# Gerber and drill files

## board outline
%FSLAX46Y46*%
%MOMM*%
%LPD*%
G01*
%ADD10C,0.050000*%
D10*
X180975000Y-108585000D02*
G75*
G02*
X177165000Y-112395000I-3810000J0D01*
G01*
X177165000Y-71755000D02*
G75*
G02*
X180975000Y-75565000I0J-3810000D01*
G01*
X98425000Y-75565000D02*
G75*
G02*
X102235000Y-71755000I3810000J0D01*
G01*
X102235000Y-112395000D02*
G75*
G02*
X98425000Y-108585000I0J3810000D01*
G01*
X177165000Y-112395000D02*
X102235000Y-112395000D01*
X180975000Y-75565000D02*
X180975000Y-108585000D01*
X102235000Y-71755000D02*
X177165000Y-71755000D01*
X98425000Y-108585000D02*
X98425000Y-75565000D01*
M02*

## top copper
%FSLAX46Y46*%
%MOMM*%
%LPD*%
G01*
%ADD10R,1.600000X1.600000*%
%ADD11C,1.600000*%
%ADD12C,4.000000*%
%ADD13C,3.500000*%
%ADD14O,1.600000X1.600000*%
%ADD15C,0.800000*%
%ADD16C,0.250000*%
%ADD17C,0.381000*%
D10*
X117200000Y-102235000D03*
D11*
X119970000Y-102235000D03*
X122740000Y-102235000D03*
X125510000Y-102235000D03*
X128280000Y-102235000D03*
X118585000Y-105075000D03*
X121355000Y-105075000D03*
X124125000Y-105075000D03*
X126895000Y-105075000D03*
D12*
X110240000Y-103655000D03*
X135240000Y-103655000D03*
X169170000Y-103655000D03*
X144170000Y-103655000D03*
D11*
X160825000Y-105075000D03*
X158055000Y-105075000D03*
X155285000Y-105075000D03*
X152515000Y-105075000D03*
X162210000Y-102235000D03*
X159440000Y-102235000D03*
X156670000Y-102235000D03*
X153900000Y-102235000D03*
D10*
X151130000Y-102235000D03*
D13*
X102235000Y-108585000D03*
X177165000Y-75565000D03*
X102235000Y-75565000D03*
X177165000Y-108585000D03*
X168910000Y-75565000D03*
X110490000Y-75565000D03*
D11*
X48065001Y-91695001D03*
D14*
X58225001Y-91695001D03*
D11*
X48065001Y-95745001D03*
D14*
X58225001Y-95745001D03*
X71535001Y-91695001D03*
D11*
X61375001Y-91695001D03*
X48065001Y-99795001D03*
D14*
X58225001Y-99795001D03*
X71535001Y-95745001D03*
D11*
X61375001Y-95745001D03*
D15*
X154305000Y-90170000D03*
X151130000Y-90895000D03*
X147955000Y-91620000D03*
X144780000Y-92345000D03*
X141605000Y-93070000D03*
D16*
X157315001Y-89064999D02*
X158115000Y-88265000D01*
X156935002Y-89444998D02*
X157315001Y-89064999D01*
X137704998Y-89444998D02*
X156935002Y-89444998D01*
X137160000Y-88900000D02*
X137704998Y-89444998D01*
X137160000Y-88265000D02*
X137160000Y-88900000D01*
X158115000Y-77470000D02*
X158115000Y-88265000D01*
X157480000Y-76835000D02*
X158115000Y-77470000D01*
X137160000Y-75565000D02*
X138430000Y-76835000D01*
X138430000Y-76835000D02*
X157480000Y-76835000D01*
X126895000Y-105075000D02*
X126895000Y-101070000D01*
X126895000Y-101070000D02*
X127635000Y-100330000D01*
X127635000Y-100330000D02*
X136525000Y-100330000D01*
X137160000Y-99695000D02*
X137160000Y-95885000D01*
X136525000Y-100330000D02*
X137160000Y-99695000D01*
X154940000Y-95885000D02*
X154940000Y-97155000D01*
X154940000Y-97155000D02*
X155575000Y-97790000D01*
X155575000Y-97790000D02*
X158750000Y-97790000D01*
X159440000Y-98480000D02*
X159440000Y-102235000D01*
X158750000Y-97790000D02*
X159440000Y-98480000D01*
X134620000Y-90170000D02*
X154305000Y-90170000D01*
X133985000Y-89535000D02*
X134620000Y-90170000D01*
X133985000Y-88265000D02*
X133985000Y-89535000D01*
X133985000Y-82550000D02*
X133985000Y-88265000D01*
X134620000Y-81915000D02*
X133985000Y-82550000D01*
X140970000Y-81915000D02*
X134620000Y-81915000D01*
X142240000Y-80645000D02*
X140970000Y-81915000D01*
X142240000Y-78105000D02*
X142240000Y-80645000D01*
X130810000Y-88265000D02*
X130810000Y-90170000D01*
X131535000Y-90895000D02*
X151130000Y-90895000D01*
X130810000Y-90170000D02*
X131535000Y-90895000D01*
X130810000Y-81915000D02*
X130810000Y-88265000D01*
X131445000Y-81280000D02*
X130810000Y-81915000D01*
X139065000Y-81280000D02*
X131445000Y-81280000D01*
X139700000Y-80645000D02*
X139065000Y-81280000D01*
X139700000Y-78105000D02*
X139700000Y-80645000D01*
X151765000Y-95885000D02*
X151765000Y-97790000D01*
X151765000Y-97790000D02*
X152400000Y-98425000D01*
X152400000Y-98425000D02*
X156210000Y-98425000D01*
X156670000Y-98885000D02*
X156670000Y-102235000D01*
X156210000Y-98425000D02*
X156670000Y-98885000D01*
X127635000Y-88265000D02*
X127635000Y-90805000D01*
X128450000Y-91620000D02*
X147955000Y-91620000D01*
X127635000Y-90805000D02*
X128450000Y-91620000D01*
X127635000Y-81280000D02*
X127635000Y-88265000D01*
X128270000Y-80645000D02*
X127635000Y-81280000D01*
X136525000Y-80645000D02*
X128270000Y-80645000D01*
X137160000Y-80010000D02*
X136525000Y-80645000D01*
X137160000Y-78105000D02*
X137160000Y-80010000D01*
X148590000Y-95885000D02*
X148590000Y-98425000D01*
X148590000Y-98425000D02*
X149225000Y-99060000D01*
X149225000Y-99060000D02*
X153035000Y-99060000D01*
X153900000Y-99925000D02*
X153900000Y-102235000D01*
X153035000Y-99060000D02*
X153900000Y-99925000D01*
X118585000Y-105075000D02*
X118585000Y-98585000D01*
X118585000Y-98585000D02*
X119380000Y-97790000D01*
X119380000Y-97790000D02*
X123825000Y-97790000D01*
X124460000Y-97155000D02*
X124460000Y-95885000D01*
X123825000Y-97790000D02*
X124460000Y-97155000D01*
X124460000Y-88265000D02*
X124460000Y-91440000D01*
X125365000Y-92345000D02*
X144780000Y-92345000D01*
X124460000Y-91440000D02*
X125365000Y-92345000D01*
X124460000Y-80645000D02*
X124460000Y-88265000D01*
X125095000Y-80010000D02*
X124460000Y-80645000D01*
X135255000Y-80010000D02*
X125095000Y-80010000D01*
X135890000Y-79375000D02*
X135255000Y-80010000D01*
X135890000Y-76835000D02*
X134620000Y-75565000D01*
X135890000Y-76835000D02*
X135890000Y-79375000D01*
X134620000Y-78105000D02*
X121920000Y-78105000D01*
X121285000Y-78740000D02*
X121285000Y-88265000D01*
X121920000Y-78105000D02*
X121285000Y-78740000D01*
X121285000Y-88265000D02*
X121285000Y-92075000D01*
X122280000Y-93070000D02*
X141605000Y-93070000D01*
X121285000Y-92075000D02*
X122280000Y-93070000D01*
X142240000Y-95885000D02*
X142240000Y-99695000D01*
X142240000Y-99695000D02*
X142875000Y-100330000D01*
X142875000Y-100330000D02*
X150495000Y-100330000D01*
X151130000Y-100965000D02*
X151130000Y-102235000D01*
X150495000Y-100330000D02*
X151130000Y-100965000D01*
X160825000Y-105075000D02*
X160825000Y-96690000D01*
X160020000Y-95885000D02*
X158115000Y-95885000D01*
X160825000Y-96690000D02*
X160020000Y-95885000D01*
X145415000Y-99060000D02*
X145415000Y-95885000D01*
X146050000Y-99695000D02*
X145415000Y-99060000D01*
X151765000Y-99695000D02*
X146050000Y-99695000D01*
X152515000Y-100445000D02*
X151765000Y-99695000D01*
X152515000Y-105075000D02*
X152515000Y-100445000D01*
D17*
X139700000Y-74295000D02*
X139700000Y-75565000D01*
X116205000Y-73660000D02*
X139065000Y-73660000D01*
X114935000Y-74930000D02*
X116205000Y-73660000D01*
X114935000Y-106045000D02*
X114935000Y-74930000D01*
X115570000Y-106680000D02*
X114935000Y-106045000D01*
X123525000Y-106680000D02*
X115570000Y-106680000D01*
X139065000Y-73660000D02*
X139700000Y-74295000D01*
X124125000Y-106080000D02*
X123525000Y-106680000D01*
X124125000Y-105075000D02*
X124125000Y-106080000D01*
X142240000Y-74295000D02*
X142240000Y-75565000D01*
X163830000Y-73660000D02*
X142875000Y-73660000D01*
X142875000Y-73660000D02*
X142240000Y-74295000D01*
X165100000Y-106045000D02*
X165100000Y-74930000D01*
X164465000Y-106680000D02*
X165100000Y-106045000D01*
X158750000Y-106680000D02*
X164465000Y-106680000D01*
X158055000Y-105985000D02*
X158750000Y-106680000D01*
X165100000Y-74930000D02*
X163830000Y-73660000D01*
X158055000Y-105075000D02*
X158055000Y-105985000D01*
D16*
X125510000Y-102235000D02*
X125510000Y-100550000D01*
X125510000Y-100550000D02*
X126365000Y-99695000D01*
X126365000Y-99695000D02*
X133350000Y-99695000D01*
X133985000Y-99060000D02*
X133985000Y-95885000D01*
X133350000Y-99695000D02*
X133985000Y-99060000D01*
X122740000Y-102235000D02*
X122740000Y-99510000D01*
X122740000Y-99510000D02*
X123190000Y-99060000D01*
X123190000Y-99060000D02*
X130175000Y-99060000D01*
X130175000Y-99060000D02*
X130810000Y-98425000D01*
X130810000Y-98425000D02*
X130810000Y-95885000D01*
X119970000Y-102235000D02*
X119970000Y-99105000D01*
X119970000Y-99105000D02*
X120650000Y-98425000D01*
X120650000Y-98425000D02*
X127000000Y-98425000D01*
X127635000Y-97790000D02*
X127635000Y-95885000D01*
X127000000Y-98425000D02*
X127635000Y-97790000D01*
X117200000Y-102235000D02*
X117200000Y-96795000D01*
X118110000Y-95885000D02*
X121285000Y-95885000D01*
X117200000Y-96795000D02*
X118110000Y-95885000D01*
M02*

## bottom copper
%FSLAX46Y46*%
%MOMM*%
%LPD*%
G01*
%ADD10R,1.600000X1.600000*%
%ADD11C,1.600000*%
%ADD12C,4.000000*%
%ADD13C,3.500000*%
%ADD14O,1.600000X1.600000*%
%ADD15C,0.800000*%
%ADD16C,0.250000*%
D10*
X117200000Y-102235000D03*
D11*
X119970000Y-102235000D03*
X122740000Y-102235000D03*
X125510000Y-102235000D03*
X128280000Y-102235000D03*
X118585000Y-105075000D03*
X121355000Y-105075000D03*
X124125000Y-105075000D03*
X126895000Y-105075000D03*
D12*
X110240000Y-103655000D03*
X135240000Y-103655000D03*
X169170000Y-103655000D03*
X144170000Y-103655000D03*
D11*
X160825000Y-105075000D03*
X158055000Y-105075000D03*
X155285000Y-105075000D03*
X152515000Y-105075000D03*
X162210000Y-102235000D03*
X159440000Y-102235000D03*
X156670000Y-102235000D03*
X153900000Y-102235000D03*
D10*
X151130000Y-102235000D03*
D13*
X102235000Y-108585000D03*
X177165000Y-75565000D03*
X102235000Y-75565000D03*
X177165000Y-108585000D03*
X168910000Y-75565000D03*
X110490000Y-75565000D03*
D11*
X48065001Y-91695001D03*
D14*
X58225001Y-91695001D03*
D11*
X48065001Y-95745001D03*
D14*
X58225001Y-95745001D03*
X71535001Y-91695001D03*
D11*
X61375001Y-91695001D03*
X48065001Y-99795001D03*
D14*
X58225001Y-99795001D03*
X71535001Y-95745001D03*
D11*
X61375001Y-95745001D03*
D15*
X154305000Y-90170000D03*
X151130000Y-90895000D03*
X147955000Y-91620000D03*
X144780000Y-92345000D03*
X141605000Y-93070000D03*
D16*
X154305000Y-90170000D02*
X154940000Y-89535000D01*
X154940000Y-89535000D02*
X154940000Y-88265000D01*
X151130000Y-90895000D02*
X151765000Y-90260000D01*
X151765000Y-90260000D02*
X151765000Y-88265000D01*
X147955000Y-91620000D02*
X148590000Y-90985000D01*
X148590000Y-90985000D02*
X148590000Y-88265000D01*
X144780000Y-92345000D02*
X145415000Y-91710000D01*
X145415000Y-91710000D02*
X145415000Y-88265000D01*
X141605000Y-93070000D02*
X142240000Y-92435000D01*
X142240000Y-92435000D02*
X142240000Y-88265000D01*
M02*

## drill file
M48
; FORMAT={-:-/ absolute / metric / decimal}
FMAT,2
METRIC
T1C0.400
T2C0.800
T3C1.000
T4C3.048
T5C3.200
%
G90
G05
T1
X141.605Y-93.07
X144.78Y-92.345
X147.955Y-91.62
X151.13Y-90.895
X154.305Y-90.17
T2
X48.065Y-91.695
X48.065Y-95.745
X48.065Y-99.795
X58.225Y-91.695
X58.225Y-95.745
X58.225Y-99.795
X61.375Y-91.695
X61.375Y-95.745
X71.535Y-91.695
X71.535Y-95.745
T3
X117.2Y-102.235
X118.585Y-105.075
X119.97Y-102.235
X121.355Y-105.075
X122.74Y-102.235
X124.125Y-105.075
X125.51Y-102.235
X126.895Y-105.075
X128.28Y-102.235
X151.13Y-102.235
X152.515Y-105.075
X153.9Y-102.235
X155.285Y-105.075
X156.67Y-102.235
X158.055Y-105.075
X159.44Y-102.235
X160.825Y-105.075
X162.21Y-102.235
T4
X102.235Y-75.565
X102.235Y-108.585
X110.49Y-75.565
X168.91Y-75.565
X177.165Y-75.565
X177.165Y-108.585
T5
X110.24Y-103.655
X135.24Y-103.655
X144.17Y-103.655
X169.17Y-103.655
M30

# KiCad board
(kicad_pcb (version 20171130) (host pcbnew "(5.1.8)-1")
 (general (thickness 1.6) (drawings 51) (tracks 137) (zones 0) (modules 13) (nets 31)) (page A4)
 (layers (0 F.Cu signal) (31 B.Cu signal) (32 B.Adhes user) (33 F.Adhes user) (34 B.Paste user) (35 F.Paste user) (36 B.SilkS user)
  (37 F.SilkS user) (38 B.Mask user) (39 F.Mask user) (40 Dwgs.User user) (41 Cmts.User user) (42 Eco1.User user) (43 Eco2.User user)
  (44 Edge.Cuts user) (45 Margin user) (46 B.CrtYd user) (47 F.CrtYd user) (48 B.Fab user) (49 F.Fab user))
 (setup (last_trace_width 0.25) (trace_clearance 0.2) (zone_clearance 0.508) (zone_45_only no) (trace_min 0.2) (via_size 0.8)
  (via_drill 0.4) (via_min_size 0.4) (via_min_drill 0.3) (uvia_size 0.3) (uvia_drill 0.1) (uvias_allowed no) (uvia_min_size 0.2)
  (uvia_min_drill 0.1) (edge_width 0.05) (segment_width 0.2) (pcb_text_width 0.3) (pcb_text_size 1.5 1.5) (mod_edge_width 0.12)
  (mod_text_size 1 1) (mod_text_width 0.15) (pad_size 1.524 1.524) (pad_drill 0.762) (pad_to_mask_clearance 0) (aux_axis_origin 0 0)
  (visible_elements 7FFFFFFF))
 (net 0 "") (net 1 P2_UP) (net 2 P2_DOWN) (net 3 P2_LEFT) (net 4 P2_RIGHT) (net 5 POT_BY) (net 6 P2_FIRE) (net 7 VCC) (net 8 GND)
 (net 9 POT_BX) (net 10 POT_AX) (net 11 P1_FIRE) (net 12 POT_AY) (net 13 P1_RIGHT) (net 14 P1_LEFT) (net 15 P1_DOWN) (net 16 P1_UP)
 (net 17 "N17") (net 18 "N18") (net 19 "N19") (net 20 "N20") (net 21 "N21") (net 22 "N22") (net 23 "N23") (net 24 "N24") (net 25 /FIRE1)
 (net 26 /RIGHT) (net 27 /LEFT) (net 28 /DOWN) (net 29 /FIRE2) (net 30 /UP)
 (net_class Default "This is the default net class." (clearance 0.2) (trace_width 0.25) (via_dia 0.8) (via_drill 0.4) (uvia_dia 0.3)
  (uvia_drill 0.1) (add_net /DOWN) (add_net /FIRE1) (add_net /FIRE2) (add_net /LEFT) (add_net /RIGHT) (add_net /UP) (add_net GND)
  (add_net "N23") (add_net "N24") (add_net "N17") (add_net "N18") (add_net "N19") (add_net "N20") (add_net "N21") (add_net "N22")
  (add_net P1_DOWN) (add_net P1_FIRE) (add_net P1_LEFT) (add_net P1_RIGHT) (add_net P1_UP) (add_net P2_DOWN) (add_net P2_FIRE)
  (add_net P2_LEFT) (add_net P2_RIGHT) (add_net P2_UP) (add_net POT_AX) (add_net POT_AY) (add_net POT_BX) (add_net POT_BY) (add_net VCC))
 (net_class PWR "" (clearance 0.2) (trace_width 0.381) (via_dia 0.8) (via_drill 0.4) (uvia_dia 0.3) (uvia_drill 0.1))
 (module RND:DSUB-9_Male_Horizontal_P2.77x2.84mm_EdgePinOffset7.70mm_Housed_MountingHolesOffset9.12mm (layer F.Cu) (at 117.2 102.235)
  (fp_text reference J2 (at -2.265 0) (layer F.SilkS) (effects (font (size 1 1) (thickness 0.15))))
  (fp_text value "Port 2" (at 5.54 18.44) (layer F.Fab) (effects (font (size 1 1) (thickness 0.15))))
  (pad 1 thru_hole rect (at 0 0) (size 1.6 1.6) (drill 1) (layers *.Cu *.Mask) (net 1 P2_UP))
  (pad 2 thru_hole circle (at 2.77 0) (size 1.6 1.6) (drill 1) (layers *.Cu *.Mask) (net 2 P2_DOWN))
  (pad 3 thru_hole circle (at 5.54 0) (size 1.6 1.6) (drill 1) (layers *.Cu *.Mask) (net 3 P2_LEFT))
  (pad 4 thru_hole circle (at 8.31 0) (size 1.6 1.6) (drill 1) (layers *.Cu *.Mask) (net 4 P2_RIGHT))
  (pad 5 thru_hole circle (at 11.08 0) (size 1.6 1.6) (drill 1) (layers *.Cu *.Mask) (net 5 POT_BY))
  (pad 6 thru_hole circle (at 1.385 2.84) (size 1.6 1.6) (drill 1) (layers *.Cu *.Mask) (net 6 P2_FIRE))
  (pad 7 thru_hole circle (at 4.155 2.84) (size 1.6 1.6) (drill 1) (layers *.Cu *.Mask) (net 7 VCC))
  (pad 8 thru_hole circle (at 6.925 2.84) (size 1.6 1.6) (drill 1) (layers *.Cu *.Mask) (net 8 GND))
  (pad 9 thru_hole circle (at 9.695 2.84) (size 1.6 1.6) (drill 1) (layers *.Cu *.Mask) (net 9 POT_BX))
  (pad 0 thru_hole circle (at -6.96 1.42) (size 4 4) (drill 3.2) (layers *.Cu *.Mask))
  (pad 0 thru_hole circle (at 18.04 1.42) (size 4 4) (drill 3.2) (layers *.Cu *.Mask)))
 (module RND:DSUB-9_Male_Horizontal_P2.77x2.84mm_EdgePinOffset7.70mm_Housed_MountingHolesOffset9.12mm (layer F.Cu) (at 151.13 102.235)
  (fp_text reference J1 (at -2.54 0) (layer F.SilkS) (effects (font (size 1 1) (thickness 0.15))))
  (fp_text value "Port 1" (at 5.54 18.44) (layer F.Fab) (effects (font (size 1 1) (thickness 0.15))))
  (pad 0 thru_hole circle (at 18.04 1.42) (size 4 4) (drill 3.2) (layers *.Cu *.Mask))
  (pad 0 thru_hole circle (at -6.96 1.42) (size 4 4) (drill 3.2) (layers *.Cu *.Mask))
  (pad 9 thru_hole circle (at 9.695 2.84) (size 1.6 1.6) (drill 1) (layers *.Cu *.Mask) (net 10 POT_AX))
  (pad 8 thru_hole circle (at 6.925 2.84) (size 1.6 1.6) (drill 1) (layers *.Cu *.Mask) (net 8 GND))
  (pad 7 thru_hole circle (at 4.155 2.84) (size 1.6 1.6) (drill 1) (layers *.Cu *.Mask) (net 7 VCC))
  (pad 6 thru_hole circle (at 1.385 2.84) (size 1.6 1.6) (drill 1) (layers *.Cu *.Mask) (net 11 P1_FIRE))
  (pad 5 thru_hole circle (at 11.08 0) (size 1.6 1.6) (drill 1) (layers *.Cu *.Mask) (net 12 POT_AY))
  (pad 4 thru_hole circle (at 8.31 0) (size 1.6 1.6) (drill 1) (layers *.Cu *.Mask) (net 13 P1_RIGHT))
  (pad 3 thru_hole circle (at 5.54 0) (size 1.6 1.6) (drill 1) (layers *.Cu *.Mask) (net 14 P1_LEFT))
  (pad 2 thru_hole circle (at 2.77 0) (size 1.6 1.6) (drill 1) (layers *.Cu *.Mask) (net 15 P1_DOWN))
  (pad 1 thru_hole rect (at 0 0) (size 1.6 1.6) (drill 1) (layers *.Cu *.Mask) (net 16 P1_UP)))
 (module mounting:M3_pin (layer F.Cu) (at 102.235 108.585)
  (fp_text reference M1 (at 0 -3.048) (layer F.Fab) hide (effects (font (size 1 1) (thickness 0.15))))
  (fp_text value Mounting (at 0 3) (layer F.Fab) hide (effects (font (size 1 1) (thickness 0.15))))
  (pad 1 thru_hole circle (at 0 0) (size 3.5 3.5) (drill 3.048) (layers *.Cu *.Mask) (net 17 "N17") (solder_mask_margin 0.8)))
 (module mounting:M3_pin (layer F.Cu) (at 177.165 75.565)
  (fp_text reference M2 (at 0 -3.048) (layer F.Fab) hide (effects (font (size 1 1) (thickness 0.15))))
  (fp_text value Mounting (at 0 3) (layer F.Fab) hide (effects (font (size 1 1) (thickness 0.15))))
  (pad 1 thru_hole circle (at 0 0) (size 3.5 3.5) (drill 3.048) (layers *.Cu *.Mask) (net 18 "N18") (solder_mask_margin 0.8)))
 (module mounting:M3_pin (layer F.Cu) (at 102.235 75.565)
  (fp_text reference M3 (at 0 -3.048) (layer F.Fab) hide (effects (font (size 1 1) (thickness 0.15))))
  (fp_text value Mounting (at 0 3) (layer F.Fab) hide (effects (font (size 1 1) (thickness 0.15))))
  (pad 1 thru_hole circle (at 0 0) (size 3.5 3.5) (drill 3.048) (layers *.Cu *.Mask) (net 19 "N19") (solder_mask_margin 0.8)))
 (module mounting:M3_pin (layer F.Cu) (at 177.165 108.585)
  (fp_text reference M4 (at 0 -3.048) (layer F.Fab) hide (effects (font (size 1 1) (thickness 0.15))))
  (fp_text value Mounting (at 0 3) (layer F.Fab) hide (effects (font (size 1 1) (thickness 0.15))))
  (pad 1 thru_hole circle (at 0 0) (size 3.5 3.5) (drill 3.048) (layers *.Cu *.Mask) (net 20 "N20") (solder_mask_margin 0.8)))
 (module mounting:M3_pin (layer F.Cu) (at 168.91 75.565)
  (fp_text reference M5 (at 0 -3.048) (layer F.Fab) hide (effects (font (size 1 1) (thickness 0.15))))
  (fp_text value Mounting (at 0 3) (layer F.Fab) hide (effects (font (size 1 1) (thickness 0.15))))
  (pad 1 thru_hole circle (at 0 0) (size 3.5 3.5) (drill 3.048) (layers *.Cu *.Mask) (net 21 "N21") (solder_mask_margin 0.8)))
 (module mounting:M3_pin (layer F.Cu) (at 110.49 75.565)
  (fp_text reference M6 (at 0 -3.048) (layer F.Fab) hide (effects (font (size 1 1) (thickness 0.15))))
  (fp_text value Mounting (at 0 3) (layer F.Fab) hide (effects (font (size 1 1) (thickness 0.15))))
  (pad 1 thru_hole circle (at 0 0) (size 3.5 3.5) (drill 3.048) (layers *.Cu *.Mask) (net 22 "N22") (solder_mask_margin 0.8)))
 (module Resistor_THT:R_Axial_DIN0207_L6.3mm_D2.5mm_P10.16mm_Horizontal (layer F.Cu) (at 48.065001 91.695001)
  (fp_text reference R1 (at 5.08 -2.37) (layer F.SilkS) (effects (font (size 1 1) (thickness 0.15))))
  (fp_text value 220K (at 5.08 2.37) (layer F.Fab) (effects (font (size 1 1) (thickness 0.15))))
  (pad 1 thru_hole circle (at 0 0) (size 1.6 1.6) (drill 0.8) (layers *.Cu *.Mask) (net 8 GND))
  (pad 2 thru_hole oval (at 10.16 0) (size 1.6 1.6) (drill 0.8) (layers *.Cu *.Mask) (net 5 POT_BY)))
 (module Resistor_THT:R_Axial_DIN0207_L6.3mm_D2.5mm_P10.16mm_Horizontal (layer F.Cu) (at 48.065001 95.745001)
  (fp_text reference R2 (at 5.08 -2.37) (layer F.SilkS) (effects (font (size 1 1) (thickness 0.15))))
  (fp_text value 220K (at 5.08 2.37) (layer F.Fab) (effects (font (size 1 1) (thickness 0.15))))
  (pad 1 thru_hole circle (at 0 0) (size 1.6 1.6) (drill 0.8) (layers *.Cu *.Mask) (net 8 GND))
  (pad 2 thru_hole oval (at 10.16 0) (size 1.6 1.6) (drill 0.8) (layers *.Cu *.Mask) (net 9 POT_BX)))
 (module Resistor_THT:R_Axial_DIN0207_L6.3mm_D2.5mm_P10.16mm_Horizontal (layer F.Cu) (at 61.375001 91.695001)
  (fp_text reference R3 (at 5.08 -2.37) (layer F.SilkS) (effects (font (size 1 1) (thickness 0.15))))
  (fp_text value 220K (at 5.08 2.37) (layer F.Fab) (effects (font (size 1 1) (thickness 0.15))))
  (pad 2 thru_hole oval (at 10.16 0) (size 1.6 1.6) (drill 0.8) (layers *.Cu *.Mask) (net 12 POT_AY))
  (pad 1 thru_hole circle (at 0 0) (size 1.6 1.6) (drill 0.8) (layers *.Cu *.Mask) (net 8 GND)))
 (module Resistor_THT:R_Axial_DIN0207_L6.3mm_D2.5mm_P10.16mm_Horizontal (layer F.Cu) (at 48.065001 99.795001)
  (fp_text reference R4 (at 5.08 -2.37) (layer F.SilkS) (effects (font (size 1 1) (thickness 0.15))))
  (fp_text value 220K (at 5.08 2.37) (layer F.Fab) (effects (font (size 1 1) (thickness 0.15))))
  (pad 1 thru_hole circle (at 0 0) (size 1.6 1.6) (drill 0.8) (layers *.Cu *.Mask) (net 8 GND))
  (pad 2 thru_hole oval (at 10.16 0) (size 1.6 1.6) (drill 0.8) (layers *.Cu *.Mask) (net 10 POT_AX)))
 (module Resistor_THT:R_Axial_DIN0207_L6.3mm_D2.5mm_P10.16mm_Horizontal (layer F.Cu) (at 61.375001 95.745001)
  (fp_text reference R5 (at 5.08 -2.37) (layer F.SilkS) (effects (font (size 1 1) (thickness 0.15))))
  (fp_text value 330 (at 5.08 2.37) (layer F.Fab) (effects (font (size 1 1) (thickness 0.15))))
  (pad 2 thru_hole oval (at 10.16 0) (size 1.6 1.6) (drill 0.8) (layers *.Cu *.Mask) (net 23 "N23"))
  (pad 1 thru_hole circle (at 0 0) (size 1.6 1.6) (drill 0.8) (layers *.Cu *.Mask) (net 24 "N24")))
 (gr_arc (start 177.165 108.585) (end 177.165 112.395) (angle -90) (layer Edge.Cuts) (width 0.05))
 (gr_arc (start 177.165 75.565) (end 180.975 75.565) (angle -90) (layer Edge.Cuts) (width 0.05))
 (gr_arc (start 102.235 75.565) (end 102.235 71.755) (angle -90) (layer Edge.Cuts) (width 0.05))
 (gr_arc (start 102.235 108.585) (end 98.425 108.585) (angle -90) (layer Edge.Cuts) (width 0.05))
 (gr_line (start 177.165 112.395) (end 102.235 112.395) (layer Edge.Cuts) (width 0.05))
 (gr_line (start 180.975 75.565) (end 180.975 108.585) (layer Edge.Cuts) (width 0.05))
 (gr_line (start 102.235 71.755) (end 177.165 71.755) (layer Edge.Cuts) (width 0.05))
 (gr_line (start 98.425 108.585) (end 98.425 75.565) (layer Edge.Cuts) (width 0.05))
 (segment (start 157.315001 89.064999) (end 158.115 88.265) (width 0.25) (layer F.Cu) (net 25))
 (segment (start 156.935002 89.444998) (end 157.315001 89.064999) (width 0.25) (layer F.Cu) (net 25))
 (segment (start 137.704998 89.444998) (end 156.935002 89.444998) (width 0.25) (layer F.Cu) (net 25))
 (segment (start 137.16 88.9) (end 137.704998 89.444998) (width 0.25) (layer F.Cu) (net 25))
 (segment (start 137.16 88.265) (end 137.16 88.9) (width 0.25) (layer F.Cu) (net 25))
 (segment (start 158.115 77.47) (end 158.115 88.265) (width 0.25) (layer F.Cu) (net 25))
 (segment (start 157.48 76.835) (end 158.115 77.47) (width 0.25) (layer F.Cu) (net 25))
 (segment (start 137.16 75.565) (end 138.43 76.835) (width 0.25) (layer F.Cu) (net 25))
 (segment (start 138.43 76.835) (end 157.48 76.835) (width 0.25) (layer F.Cu) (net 25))
 (segment (start 126.895 105.075) (end 126.895 101.07) (width 0.25) (layer F.Cu) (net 9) (status 10))
 (segment (start 126.895 101.07) (end 127.635 100.33) (width 0.25) (layer F.Cu) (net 9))
 (segment (start 127.635 100.33) (end 136.525 100.33) (width 0.25) (layer F.Cu) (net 9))
 (segment (start 137.16 99.695) (end 137.16 95.885) (width 0.25) (layer F.Cu) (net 9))
 (segment (start 136.525 100.33) (end 137.16 99.695) (width 0.25) (layer F.Cu) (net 9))
 (segment (start 154.94 95.885) (end 154.94 97.155) (width 0.25) (layer F.Cu) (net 13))
 (segment (start 154.94 97.155) (end 155.575 97.79) (width 0.25) (layer F.Cu) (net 13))
 (segment (start 155.575 97.79) (end 158.75 97.79) (width 0.25) (layer F.Cu) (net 13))
 (segment (start 159.44 98.48) (end 159.44 102.235) (width 0.25) (layer F.Cu) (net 13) (status 20))
 (segment (start 158.75 97.79) (end 159.44 98.48) (width 0.25) (layer F.Cu) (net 13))
 (via (at 154.305 90.17) (size 0.8) (drill 0.4) (layers F.Cu B.Cu) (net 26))
 (segment (start 154.305 90.17) (end 154.94 89.535) (width 0.25) (layer B.Cu) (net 26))
 (segment (start 154.94 89.535) (end 154.94 88.265) (width 0.25) (layer B.Cu) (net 26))
 (segment (start 134.62 90.17) (end 154.305 90.17) (width 0.25) (layer F.Cu) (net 26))
 (segment (start 133.985 89.535) (end 134.62 90.17) (width 0.25) (layer F.Cu) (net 26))
 (segment (start 133.985 88.265) (end 133.985 89.535) (width 0.25) (layer F.Cu) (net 26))
 (segment (start 133.985 82.55) (end 133.985 88.265) (width 0.25) (layer F.Cu) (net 26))
 (segment (start 134.62 81.915) (end 133.985 82.55) (width 0.25) (layer F.Cu) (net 26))
 (segment (start 140.97 81.915) (end 134.62 81.915) (width 0.25) (layer F.Cu) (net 26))
 (segment (start 142.24 80.645) (end 140.97 81.915) (width 0.25) (layer F.Cu) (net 26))
 (segment (start 142.24 78.105) (end 142.24 80.645) (width 0.25) (layer F.Cu) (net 26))
 (segment (start 130.81 88.265) (end 130.81 90.17) (width 0.25) (layer F.Cu) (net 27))
 (via (at 151.13 90.895) (size 0.8) (drill 0.4) (layers F.Cu B.Cu) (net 27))
 (segment (start 131.535 90.895) (end 151.13 90.895) (width 0.25) (layer F.Cu) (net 27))
 (segment (start 130.81 90.17) (end 131.535 90.895) (width 0.25) (layer F.Cu) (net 27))
 (segment (start 151.13 90.895) (end 151.765 90.26) (width 0.25) (layer B.Cu) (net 27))
 (segment (start 151.765 90.26) (end 151.765 88.265) (width 0.25) (layer B.Cu) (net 27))
 (segment (start 130.81 81.915) (end 130.81 88.265) (width 0.25) (layer F.Cu) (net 27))
 (segment (start 131.445 81.28) (end 130.81 81.915) (width 0.25) (layer F.Cu) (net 27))
 (segment (start 139.065 81.28) (end 131.445 81.28) (width 0.25) (layer F.Cu) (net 27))
 (segment (start 139.7 80.645) (end 139.065 81.28) (width 0.25) (layer F.Cu) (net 27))
 (segment (start 139.7 78.105) (end 139.7 80.645) (width 0.25) (layer F.Cu) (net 27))
 (segment (start 151.765 95.885) (end 151.765 97.79) (width 0.25) (layer F.Cu) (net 14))
 (segment (start 151.765 97.79) (end 152.4 98.425) (width 0.25) (layer F.Cu) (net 14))
 (segment (start 152.4 98.425) (end 156.21 98.425) (width 0.25) (layer F.Cu) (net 14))
 (segment (start 156.67 98.885) (end 156.67 102.235) (width 0.25) (layer F.Cu) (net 14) (status 20))
 (segment (start 156.21 98.425) (end 156.67 98.885) (width 0.25) (layer F.Cu) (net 14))
 (segment (start 127.635 88.265) (end 127.635 90.805) (width 0.25) (layer F.Cu) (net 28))
 (via (at 147.955 91.62) (size 0.8) (drill 0.4) (layers F.Cu B.Cu) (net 28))
 (segment (start 128.45 91.62) (end 147.955 91.62) (width 0.25) (layer F.Cu) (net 28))
 (segment (start 127.635 90.805) (end 128.45 91.62) (width 0.25) (layer F.Cu) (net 28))
 (segment (start 147.955 91.62) (end 148.59 90.985) (width 0.25) (layer B.Cu) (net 28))
 (segment (start 148.59 90.985) (end 148.59 88.265) (width 0.25) (layer B.Cu) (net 28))
 (segment (start 127.635 81.28) (end 127.635 88.265) (width 0.25) (layer F.Cu) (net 28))
 (segment (start 128.27 80.645) (end 127.635 81.28) (width 0.25) (layer F.Cu) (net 28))
 (segment (start 136.525 80.645) (end 128.27 80.645) (width 0.25) (layer F.Cu) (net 28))
 (segment (start 137.16 80.01) (end 136.525 80.645) (width 0.25) (layer F.Cu) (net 28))
 (segment (start 137.16 78.105) (end 137.16 80.01) (width 0.25) (layer F.Cu) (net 28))
 (segment (start 148.59 95.885) (end 148.59 98.425) (width 0.25) (layer F.Cu) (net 15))
 (segment (start 148.59 98.425) (end 149.225 99.06) (width 0.25) (layer F.Cu) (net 15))
 (segment (start 149.225 99.06) (end 153.035 99.06) (width 0.25) (layer F.Cu) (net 15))
 (segment (start 153.9 99.925) (end 153.9 102.235) (width 0.25) (layer F.Cu) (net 15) (status 20))
 (segment (start 153.035 99.06) (end 153.9 99.925) (width 0.25) (layer F.Cu) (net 15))
 (segment (start 118.585 105.075) (end 118.585 98.585) (width 0.25) (layer F.Cu) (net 6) (status 10))
 (segment (start 118.585 98.585) (end 119.38 97.79) (width 0.25) (layer F.Cu) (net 6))
 (segment (start 119.38 97.79) (end 123.825 97.79) (width 0.25) (layer F.Cu) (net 6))
 (segment (start 124.46 97.155) (end 124.46 95.885) (width 0.25) (layer F.Cu) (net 6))
 (segment (start 123.825 97.79) (end 124.46 97.155) (width 0.25) (layer F.Cu) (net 6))
 (segment (start 124.46 88.265) (end 124.46 91.44) (width 0.25) (layer F.Cu) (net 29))
 (via (at 144.78 92.345) (size 0.8) (drill 0.4) (layers F.Cu B.Cu) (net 29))
 (segment (start 125.365 92.345) (end 144.78 92.345) (width 0.25) (layer F.Cu) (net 29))
 (segment (start 124.46 91.44) (end 125.365 92.345) (width 0.25) (layer F.Cu) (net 29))
 (segment (start 144.78 92.345) (end 145.415 91.71) (width 0.25) (layer B.Cu) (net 29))
 (segment (start 145.415 91.71) (end 145.415 88.265) (width 0.25) (layer B.Cu) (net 29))
 (segment (start 124.46 80.645) (end 124.46 88.265) (width 0.25) (layer F.Cu) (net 29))
 (segment (start 125.095 80.01) (end 124.46 80.645) (width 0.25) (layer F.Cu) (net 29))
 (segment (start 135.255 80.01) (end 125.095 80.01) (width 0.25) (layer F.Cu) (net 29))
 (segment (start 135.89 79.375) (end 135.255 80.01) (width 0.25) (layer F.Cu) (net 29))
 (segment (start 135.89 76.835) (end 134.62 75.565) (width 0.25) (layer F.Cu) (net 29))
 (segment (start 135.89 76.835) (end 135.89 79.375) (width 0.25) (layer F.Cu) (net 29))
 (segment (start 134.62 78.105) (end 121.92 78.105) (width 0.25) (layer F.Cu) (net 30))
 (segment (start 121.285 78.74) (end 121.285 88.265) (width 0.25) (layer F.Cu) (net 30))
 (segment (start 121.92 78.105) (end 121.285 78.74) (width 0.25) (layer F.Cu) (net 30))
 (segment (start 121.285 88.265) (end 121.285 92.075) (width 0.25) (layer F.Cu) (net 30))
 (via (at 141.605 93.07) (size 0.8) (drill 0.4) (layers F.Cu B.Cu) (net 30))
 (segment (start 122.28 93.07) (end 141.605 93.07) (width 0.25) (layer F.Cu) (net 30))
 (segment (start 121.285 92.075) (end 122.28 93.07) (width 0.25) (layer F.Cu) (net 30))
 (segment (start 141.605 93.07) (end 142.24 92.435) (width 0.25) (layer B.Cu) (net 30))
 (segment (start 142.24 92.435) (end 142.24 88.265) (width 0.25) (layer B.Cu) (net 30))
 (segment (start 142.24 95.885) (end 142.24 99.695) (width 0.25) (layer F.Cu) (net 16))
 (segment (start 142.24 99.695) (end 142.875 100.33) (width 0.25) (layer F.Cu) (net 16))
 (segment (start 142.875 100.33) (end 150.495 100.33) (width 0.25) (layer F.Cu) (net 16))
 (segment (start 151.13 100.965) (end 151.13 102.235) (width 0.25) (layer F.Cu) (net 16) (status 20))
 (segment (start 150.495 100.33) (end 151.13 100.965) (width 0.25) (layer F.Cu) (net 16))
 (segment (start 160.825 105.075) (end 160.825 96.69) (width 0.25) (layer F.Cu) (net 10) (status 10))
 (segment (start 160.02 95.885) (end 158.115 95.885) (width 0.25) (layer F.Cu) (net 10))
 (segment (start 160.825 96.69) (end 160.02 95.885) (width 0.25) (layer F.Cu) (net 10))
 (segment (start 145.415 99.06) (end 145.415 95.885) (width 0.25) (layer F.Cu) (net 11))
 (segment (start 146.05 99.695) (end 145.415 99.06) (width 0.25) (layer F.Cu) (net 11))
 (segment (start 151.765 99.695) (end 146.05 99.695) (width 0.25) (layer F.Cu) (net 11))
 (segment (start 152.515 100.445) (end 151.765 99.695) (width 0.25) (layer F.Cu) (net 11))
 (segment (start 152.515 105.075) (end 152.515 100.445) (width 0.25) (layer F.Cu) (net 11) (status 10))
 (segment (start 139.7 74.295) (end 139.7 75.565) (width 0.381) (layer F.Cu) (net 8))
 (segment (start 116.205 73.66) (end 139.065 73.66) (width 0.381) (layer F.Cu) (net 8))
 (segment (start 114.935 74.93) (end 116.205 73.66) (width 0.381) (layer F.Cu) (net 8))
 (segment (start 114.935 106.045) (end 114.935 74.93) (width 0.381) (layer F.Cu) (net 8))
 (segment (start 115.57 106.68) (end 114.935 106.045) (width 0.381) (layer F.Cu) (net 8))
 (segment (start 123.525 106.68) (end 115.57 106.68) (width 0.381) (layer F.Cu) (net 8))
 (segment (start 139.065 73.66) (end 139.7 74.295) (width 0.381) (layer F.Cu) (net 8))
 (segment (start 124.125 106.08) (end 123.525 106.68) (width 0.381) (layer F.Cu) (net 8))
 (segment (start 124.125 105.075) (end 124.125 106.08) (width 0.381) (layer F.Cu) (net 8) (status 10))
 (segment (start 142.24 74.295) (end 142.24 75.565) (width 0.381) (layer F.Cu) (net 8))
 (segment (start 163.83 73.66) (end 142.875 73.66) (width 0.381) (layer F.Cu) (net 8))
 (segment (start 142.875 73.66) (end 142.24 74.295) (width 0.381) (layer F.Cu) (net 8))
 (segment (start 165.1 106.045) (end 165.1 74.93) (width 0.381) (layer F.Cu) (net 8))
 (segment (start 164.465 106.68) (end 165.1 106.045) (width 0.381) (layer F.Cu) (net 8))
 (segment (start 158.75 106.68) (end 164.465 106.68) (width 0.381) (layer F.Cu) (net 8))
 (segment (start 158.055 105.985) (end 158.75 106.68) (width 0.381) (layer F.Cu) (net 8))
 (segment (start 165.1 74.93) (end 163.83 73.66) (width 0.381) (layer F.Cu) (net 8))
 (segment (start 158.055 105.075) (end 158.055 105.985) (width 0.381) (layer F.Cu) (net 8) (status 10))
 (segment (start 125.51 102.235) (end 125.51 100.55) (width 0.25) (layer F.Cu) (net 4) (status 10))
 (segment (start 125.51 100.55) (end 126.365 99.695) (width 0.25) (layer F.Cu) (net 4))
 (segment (start 126.365 99.695) (end 133.35 99.695) (width 0.25) (layer F.Cu) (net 4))
 (segment (start 133.985 99.06) (end 133.985 95.885) (width 0.25) (layer F.Cu) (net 4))
 (segment (start 133.35 99.695) (end 133.985 99.06) (width 0.25) (layer F.Cu) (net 4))
 (segment (start 122.74 102.235) (end 122.74 99.51) (width 0.25) (layer F.Cu) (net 3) (status 10))
 (segment (start 122.74 99.51) (end 123.19 99.06) (width 0.25) (layer F.Cu) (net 3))
 (segment (start 123.19 99.06) (end 130.175 99.06) (width 0.25) (layer F.Cu) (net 3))
 (segment (start 130.175 99.06) (end 130.81 98.425) (width 0.25) (layer F.Cu) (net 3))
 (segment (start 130.81 98.425) (end 130.81 95.885) (width 0.25) (layer F.Cu) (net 3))
 (segment (start 119.97 102.235) (end 119.97 99.105) (width 0.25) (layer F.Cu) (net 2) (status 10))
 (segment (start 119.97 99.105) (end 120.65 98.425) (width 0.25) (layer F.Cu) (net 2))
 (segment (start 120.65 98.425) (end 127 98.425) (width 0.25) (layer F.Cu) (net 2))
 (segment (start 127.635 97.79) (end 127.635 95.885) (width 0.25) (layer F.Cu) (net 2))
 (segment (start 127 98.425) (end 127.635 97.79) (width 0.25) (layer F.Cu) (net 2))
 (segment (start 117.2 102.235) (end 117.2 96.795) (width 0.25) (layer F.Cu) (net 1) (status 10))
 (segment (start 118.11 95.885) (end 121.285 95.885) (width 0.25) (layer F.Cu) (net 1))
 (segment (start 117.2 96.795) (end 118.11 95.885) (width 0.25) (layer F.Cu) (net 1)))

